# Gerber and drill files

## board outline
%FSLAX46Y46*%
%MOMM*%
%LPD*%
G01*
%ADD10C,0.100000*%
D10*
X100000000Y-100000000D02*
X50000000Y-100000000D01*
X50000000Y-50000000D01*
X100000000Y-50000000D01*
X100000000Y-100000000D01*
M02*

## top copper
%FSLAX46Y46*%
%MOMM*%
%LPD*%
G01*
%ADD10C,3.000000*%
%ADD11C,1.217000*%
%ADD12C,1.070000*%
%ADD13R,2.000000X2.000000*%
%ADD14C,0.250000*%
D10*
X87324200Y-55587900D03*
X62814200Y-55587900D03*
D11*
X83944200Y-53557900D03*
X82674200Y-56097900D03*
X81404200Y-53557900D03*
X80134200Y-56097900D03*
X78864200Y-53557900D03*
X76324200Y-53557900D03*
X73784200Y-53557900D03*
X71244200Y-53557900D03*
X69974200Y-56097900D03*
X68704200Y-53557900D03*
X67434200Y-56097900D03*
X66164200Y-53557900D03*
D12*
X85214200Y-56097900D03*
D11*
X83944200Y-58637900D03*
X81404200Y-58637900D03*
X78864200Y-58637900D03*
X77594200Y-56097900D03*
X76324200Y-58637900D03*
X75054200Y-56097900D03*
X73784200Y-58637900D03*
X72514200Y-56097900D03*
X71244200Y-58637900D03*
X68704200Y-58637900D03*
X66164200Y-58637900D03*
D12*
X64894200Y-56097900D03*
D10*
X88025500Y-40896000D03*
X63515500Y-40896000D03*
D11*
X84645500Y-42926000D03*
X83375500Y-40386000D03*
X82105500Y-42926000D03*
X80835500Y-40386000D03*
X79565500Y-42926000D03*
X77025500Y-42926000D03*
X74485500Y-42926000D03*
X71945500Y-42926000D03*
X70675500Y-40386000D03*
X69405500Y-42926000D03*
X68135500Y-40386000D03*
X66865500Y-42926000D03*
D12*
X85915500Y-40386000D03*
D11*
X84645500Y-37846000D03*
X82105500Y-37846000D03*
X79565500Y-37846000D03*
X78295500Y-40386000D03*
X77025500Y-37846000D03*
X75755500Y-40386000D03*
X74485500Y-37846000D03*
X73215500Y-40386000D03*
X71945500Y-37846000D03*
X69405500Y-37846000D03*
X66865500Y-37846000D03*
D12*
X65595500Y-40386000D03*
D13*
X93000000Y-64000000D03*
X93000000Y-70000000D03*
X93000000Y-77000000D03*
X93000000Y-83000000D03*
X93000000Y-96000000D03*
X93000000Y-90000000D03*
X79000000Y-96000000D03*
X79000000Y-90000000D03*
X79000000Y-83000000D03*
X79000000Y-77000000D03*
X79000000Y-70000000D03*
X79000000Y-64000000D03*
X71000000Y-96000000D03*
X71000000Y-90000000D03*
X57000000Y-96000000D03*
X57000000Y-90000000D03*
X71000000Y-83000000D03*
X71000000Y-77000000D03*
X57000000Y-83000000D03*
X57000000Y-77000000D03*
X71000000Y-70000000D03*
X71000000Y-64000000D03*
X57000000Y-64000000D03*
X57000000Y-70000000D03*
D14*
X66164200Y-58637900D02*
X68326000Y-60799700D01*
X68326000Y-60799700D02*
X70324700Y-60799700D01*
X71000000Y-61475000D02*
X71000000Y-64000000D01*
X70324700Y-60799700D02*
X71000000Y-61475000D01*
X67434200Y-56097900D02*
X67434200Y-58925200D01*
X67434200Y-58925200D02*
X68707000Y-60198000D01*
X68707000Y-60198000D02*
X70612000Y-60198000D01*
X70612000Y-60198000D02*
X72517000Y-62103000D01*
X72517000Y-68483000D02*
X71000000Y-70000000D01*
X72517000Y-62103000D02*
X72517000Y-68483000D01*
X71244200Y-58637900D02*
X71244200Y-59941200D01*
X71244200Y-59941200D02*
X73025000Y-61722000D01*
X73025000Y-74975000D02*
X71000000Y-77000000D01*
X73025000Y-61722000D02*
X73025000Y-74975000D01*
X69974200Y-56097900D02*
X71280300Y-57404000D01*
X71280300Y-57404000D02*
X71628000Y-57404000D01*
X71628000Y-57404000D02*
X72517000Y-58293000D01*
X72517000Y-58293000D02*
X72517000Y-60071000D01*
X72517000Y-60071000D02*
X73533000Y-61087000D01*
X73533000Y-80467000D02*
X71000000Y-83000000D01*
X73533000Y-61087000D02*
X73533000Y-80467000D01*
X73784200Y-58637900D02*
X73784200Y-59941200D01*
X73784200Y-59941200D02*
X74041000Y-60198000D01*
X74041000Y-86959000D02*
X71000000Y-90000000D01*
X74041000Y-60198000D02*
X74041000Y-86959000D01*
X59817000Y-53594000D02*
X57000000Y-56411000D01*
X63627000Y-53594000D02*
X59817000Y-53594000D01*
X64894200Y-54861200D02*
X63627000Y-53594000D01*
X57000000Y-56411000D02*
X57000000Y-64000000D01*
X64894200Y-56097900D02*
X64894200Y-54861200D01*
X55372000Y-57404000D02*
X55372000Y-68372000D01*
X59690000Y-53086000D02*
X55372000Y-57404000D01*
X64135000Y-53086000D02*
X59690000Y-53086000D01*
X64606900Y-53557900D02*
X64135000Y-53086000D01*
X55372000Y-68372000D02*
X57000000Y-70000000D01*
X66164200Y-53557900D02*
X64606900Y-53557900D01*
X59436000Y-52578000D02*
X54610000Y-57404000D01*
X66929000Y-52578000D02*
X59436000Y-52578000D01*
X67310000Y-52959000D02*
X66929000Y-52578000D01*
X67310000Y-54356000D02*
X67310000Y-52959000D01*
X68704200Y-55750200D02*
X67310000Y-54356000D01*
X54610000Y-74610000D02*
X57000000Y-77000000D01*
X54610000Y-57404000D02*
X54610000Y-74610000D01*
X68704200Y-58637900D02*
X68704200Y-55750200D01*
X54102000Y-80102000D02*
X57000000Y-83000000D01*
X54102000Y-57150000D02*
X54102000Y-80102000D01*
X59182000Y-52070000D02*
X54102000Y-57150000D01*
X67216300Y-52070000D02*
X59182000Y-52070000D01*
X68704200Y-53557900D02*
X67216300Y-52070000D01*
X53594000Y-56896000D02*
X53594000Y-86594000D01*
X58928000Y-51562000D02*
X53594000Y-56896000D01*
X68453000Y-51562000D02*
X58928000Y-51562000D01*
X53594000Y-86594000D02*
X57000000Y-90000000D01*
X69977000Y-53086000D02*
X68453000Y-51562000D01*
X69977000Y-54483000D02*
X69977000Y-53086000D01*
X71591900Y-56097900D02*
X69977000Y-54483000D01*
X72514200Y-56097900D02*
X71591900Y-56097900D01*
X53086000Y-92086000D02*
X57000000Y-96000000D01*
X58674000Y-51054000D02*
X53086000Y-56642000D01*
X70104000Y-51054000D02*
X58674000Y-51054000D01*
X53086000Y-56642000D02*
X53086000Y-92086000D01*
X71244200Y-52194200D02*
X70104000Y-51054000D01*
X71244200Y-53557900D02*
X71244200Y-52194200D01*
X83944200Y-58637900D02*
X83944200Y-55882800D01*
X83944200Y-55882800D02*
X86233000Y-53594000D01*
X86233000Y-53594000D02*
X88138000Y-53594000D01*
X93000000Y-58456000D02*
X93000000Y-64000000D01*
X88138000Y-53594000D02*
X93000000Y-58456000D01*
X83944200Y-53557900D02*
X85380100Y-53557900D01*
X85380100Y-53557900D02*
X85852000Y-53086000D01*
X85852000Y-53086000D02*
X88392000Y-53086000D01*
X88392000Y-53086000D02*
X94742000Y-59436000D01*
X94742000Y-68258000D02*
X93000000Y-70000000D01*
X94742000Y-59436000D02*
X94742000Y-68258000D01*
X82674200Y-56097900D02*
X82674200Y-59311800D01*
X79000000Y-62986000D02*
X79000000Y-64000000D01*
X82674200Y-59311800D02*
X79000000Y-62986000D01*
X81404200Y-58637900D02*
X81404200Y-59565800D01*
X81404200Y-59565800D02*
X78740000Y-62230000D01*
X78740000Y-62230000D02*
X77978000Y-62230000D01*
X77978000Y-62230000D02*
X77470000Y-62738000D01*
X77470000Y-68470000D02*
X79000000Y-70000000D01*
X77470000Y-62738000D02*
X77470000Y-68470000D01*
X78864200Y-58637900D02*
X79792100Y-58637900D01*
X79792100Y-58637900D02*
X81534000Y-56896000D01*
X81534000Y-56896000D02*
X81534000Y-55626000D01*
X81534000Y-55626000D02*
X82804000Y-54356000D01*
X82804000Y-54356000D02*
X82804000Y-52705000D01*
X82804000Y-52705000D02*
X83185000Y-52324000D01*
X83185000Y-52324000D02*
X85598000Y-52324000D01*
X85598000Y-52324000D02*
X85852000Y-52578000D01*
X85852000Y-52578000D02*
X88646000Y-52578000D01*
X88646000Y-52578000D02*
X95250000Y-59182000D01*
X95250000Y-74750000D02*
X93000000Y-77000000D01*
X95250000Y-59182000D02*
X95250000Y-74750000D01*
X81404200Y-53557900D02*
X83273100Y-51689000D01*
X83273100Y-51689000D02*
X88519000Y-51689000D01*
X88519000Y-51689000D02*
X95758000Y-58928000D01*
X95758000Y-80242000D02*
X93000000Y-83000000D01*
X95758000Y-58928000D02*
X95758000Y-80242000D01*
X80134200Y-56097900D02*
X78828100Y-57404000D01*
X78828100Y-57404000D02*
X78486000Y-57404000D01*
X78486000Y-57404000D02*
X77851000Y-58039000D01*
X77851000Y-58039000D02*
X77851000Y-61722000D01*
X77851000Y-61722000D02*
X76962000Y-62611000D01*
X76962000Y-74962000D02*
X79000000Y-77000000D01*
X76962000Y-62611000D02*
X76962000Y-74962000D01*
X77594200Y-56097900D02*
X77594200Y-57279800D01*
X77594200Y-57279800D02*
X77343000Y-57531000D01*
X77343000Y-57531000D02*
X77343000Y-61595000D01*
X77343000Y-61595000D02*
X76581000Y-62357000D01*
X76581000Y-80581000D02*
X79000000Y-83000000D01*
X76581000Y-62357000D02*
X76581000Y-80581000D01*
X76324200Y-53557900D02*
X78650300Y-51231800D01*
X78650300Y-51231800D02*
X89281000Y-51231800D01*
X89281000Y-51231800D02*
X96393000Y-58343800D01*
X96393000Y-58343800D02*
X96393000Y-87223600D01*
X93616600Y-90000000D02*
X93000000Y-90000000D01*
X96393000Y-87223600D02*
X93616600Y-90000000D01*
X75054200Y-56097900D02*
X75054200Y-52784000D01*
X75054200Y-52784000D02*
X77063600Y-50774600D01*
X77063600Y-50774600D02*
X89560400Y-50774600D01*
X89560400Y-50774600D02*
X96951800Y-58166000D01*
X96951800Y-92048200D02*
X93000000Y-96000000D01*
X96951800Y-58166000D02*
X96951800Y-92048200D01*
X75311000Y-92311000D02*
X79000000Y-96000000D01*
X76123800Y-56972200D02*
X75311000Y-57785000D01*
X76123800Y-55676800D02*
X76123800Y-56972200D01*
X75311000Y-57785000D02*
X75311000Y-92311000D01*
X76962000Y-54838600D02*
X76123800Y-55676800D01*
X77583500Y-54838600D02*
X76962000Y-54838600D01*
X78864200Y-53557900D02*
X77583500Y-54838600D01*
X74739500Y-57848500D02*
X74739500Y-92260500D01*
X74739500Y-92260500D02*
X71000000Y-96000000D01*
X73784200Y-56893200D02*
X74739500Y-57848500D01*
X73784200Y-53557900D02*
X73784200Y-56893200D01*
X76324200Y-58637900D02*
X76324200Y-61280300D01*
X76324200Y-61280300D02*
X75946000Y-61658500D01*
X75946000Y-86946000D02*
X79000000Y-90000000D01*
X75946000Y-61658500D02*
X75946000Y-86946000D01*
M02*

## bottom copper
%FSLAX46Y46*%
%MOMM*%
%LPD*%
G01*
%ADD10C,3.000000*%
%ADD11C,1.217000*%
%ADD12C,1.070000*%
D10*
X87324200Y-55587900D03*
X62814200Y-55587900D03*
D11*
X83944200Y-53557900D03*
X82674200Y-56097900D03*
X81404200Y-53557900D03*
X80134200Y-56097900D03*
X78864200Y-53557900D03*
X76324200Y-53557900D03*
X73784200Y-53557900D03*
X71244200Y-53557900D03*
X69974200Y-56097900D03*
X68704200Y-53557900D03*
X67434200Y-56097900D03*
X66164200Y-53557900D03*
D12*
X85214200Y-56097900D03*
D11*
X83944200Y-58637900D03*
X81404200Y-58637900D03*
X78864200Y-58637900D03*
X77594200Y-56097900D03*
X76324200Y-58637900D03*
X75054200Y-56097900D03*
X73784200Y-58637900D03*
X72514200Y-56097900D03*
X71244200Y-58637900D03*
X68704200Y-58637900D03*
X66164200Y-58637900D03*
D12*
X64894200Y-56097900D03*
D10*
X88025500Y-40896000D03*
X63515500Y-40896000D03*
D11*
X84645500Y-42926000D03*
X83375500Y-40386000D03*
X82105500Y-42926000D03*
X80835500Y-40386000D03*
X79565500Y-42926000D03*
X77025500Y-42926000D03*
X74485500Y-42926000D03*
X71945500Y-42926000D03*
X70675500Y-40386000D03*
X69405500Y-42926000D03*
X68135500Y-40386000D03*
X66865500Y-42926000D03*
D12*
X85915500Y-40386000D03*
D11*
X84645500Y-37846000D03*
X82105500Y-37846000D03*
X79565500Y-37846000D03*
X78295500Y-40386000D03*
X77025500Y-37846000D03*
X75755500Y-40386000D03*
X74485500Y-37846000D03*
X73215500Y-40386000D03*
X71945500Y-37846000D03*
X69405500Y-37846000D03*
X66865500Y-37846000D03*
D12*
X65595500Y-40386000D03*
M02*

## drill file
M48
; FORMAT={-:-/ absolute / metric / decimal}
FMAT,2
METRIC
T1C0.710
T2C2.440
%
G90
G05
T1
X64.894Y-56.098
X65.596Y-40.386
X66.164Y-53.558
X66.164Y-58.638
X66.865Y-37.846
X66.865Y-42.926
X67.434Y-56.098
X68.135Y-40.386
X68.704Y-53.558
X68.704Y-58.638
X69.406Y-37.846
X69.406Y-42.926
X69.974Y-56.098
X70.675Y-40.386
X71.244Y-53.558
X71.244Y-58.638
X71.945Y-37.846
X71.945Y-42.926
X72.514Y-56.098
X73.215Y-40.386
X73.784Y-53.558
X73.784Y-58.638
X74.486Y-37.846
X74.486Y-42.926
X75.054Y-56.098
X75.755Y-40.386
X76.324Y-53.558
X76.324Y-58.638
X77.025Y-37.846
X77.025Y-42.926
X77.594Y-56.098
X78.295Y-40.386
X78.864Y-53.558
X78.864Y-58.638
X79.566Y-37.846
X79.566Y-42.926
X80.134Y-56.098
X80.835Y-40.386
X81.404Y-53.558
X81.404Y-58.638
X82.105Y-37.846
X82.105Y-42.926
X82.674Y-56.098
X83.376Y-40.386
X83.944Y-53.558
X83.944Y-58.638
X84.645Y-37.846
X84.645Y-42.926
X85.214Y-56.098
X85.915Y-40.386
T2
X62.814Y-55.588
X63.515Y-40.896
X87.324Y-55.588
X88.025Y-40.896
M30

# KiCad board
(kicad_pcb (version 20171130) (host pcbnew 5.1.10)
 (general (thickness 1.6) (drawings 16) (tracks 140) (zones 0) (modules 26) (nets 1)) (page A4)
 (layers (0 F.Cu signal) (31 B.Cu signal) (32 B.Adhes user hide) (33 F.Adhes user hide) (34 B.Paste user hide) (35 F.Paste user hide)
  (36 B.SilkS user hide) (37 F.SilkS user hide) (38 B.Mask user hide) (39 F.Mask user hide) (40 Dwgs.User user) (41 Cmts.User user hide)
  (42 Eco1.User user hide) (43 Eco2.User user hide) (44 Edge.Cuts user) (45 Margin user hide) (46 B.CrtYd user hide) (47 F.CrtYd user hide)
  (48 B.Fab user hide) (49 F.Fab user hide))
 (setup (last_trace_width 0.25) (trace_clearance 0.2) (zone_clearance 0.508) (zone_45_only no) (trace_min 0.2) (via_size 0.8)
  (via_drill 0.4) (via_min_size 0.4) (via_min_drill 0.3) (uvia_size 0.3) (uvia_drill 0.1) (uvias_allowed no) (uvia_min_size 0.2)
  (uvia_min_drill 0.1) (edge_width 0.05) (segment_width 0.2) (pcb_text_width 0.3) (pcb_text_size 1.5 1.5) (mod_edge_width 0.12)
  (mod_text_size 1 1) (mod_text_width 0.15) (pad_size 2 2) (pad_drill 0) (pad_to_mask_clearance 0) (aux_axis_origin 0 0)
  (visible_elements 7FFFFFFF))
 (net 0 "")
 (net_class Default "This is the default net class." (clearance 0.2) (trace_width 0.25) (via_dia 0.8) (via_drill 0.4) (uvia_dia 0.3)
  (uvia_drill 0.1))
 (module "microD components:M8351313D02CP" (layer F.Cu) (at 64.8942 56.0979 180)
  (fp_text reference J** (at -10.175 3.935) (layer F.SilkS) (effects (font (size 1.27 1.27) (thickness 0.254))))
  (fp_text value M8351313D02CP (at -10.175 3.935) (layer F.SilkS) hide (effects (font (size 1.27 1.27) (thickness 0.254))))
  (pad MH2 thru_hole circle (at -22.43 0.51 180) (size 3 3) (drill 2.44) (layers *.Cu *.Mask))
  (pad MH1 thru_hole circle (at 2.08 0.51 180) (size 3 3) (drill 2.44) (layers *.Cu *.Mask))
  (pad 25 thru_hole circle (at -19.05 2.54 180) (size 1.217 1.217) (drill 0.71) (layers *.Cu *.Mask))
  (pad 24 thru_hole circle (at -17.78 0 180) (size 1.217 1.217) (drill 0.71) (layers *.Cu *.Mask))
  (pad 23 thru_hole circle (at -16.51 2.54 180) (size 1.217 1.217) (drill 0.71) (layers *.Cu *.Mask))
  (pad 22 thru_hole circle (at -15.24 0 180) (size 1.217 1.217) (drill 0.71) (layers *.Cu *.Mask))
  (pad 21 thru_hole circle (at -13.97 2.54 180) (size 1.217 1.217) (drill 0.71) (layers *.Cu *.Mask))
  (pad 20 thru_hole circle (at -11.43 2.54 180) (size 1.217 1.217) (drill 0.71) (layers *.Cu *.Mask))
  (pad 19 thru_hole circle (at -8.89 2.54 180) (size 1.217 1.217) (drill 0.71) (layers *.Cu *.Mask))
  (pad 18 thru_hole circle (at -6.35 2.54 180) (size 1.217 1.217) (drill 0.71) (layers *.Cu *.Mask))
  (pad 17 thru_hole circle (at -5.08 0 180) (size 1.217 1.217) (drill 0.71) (layers *.Cu *.Mask))
  (pad 16 thru_hole circle (at -3.81 2.54 180) (size 1.217 1.217) (drill 0.71) (layers *.Cu *.Mask))
  (pad 15 thru_hole circle (at -2.54 0 180) (size 1.217 1.217) (drill 0.71) (layers *.Cu *.Mask))
  (pad 14 thru_hole circle (at -1.27 2.54 180) (size 1.217 1.217) (drill 0.71) (layers *.Cu *.Mask))
  (pad 13 thru_hole circle (at -20.32 0 180) (size 1.07 1.07) (drill 0.71) (layers *.Cu *.Mask))
  (pad 12 thru_hole circle (at -19.05 -2.54 180) (size 1.217 1.217) (drill 0.71) (layers *.Cu *.Mask))
  (pad 11 thru_hole circle (at -16.51 -2.54 180) (size 1.217 1.217) (drill 0.71) (layers *.Cu *.Mask))
  (pad 10 thru_hole circle (at -13.97 -2.54 180) (size 1.217 1.217) (drill 0.71) (layers *.Cu *.Mask))
  (pad 9 thru_hole circle (at -12.7 0 180) (size 1.217 1.217) (drill 0.71) (layers *.Cu *.Mask))
  (pad 8 thru_hole circle (at -11.43 -2.54 180) (size 1.217 1.217) (drill 0.71) (layers *.Cu *.Mask))
  (pad 7 thru_hole circle (at -10.16 0 180) (size 1.217 1.217) (drill 0.71) (layers *.Cu *.Mask))
  (pad 6 thru_hole circle (at -8.89 -2.54 180) (size 1.217 1.217) (drill 0.71) (layers *.Cu *.Mask))
  (pad 5 thru_hole circle (at -7.62 0 180) (size 1.217 1.217) (drill 0.71) (layers *.Cu *.Mask))
  (pad 4 thru_hole circle (at -6.35 -2.54 180) (size 1.217 1.217) (drill 0.71) (layers *.Cu *.Mask))
  (pad 3 thru_hole circle (at -3.81 -2.54 180) (size 1.217 1.217) (drill 0.71) (layers *.Cu *.Mask))
  (pad 2 thru_hole circle (at -1.27 -2.54 180) (size 1.217 1.217) (drill 0.71) (layers *.Cu *.Mask))
  (pad 1 thru_hole circle (at 0 0 180) (size 1.07 1.07) (drill 0.71) (layers *.Cu *.Mask)))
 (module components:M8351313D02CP (layer B.Cu) (at 65.5955 40.386 180)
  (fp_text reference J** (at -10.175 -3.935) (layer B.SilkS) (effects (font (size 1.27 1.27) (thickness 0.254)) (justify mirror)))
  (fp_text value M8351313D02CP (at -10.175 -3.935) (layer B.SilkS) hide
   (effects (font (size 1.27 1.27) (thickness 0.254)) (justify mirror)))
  (pad MH2 thru_hole circle (at -22.43 -0.51 180) (size 3 3) (drill 2.44) (layers *.Cu *.Mask))
  (pad MH1 thru_hole circle (at 2.08 -0.51 180) (size 3 3) (drill 2.44) (layers *.Cu *.Mask))
  (pad 25 thru_hole circle (at -19.05 -2.54 180) (size 1.217 1.217) (drill 0.71) (layers *.Cu *.Mask))
  (pad 24 thru_hole circle (at -17.78 0 180) (size 1.217 1.217) (drill 0.71) (layers *.Cu *.Mask))
  (pad 23 thru_hole circle (at -16.51 -2.54 180) (size 1.217 1.217) (drill 0.71) (layers *.Cu *.Mask))
  (pad 22 thru_hole circle (at -15.24 0 180) (size 1.217 1.217) (drill 0.71) (layers *.Cu *.Mask))
  (pad 21 thru_hole circle (at -13.97 -2.54 180) (size 1.217 1.217) (drill 0.71) (layers *.Cu *.Mask))
  (pad 20 thru_hole circle (at -11.43 -2.54 180) (size 1.217 1.217) (drill 0.71) (layers *.Cu *.Mask))
  (pad 19 thru_hole circle (at -8.89 -2.54 180) (size 1.217 1.217) (drill 0.71) (layers *.Cu *.Mask))
  (pad 18 thru_hole circle (at -6.35 -2.54 180) (size 1.217 1.217) (drill 0.71) (layers *.Cu *.Mask))
  (pad 17 thru_hole circle (at -5.08 0 180) (size 1.217 1.217) (drill 0.71) (layers *.Cu *.Mask))
  (pad 16 thru_hole circle (at -3.81 -2.54 180) (size 1.217 1.217) (drill 0.71) (layers *.Cu *.Mask))
  (pad 15 thru_hole circle (at -2.54 0 180) (size 1.217 1.217) (drill 0.71) (layers *.Cu *.Mask))
  (pad 14 thru_hole circle (at -1.27 -2.54 180) (size 1.217 1.217) (drill 0.71) (layers *.Cu *.Mask))
  (pad 13 thru_hole circle (at -20.32 0 180) (size 1.07 1.07) (drill 0.71) (layers *.Cu *.Mask))
  (pad 12 thru_hole circle (at -19.05 2.54 180) (size 1.217 1.217) (drill 0.71) (layers *.Cu *.Mask))
  (pad 11 thru_hole circle (at -16.51 2.54 180) (size 1.217 1.217) (drill 0.71) (layers *.Cu *.Mask))
  (pad 10 thru_hole circle (at -13.97 2.54 180) (size 1.217 1.217) (drill 0.71) (layers *.Cu *.Mask))
  (pad 9 thru_hole circle (at -12.7 0 180) (size 1.217 1.217) (drill 0.71) (layers *.Cu *.Mask))
  (pad 8 thru_hole circle (at -11.43 2.54 180) (size 1.217 1.217) (drill 0.71) (layers *.Cu *.Mask))
  (pad 7 thru_hole circle (at -10.16 0 180) (size 1.217 1.217) (drill 0.71) (layers *.Cu *.Mask))
  (pad 6 thru_hole circle (at -8.89 2.54 180) (size 1.217 1.217) (drill 0.71) (layers *.Cu *.Mask))
  (pad 5 thru_hole circle (at -7.62 0 180) (size 1.217 1.217) (drill 0.71) (layers *.Cu *.Mask))
  (pad 4 thru_hole circle (at -6.35 2.54 180) (size 1.217 1.217) (drill 0.71) (layers *.Cu *.Mask))
  (pad 3 thru_hole circle (at -3.81 2.54 180) (size 1.217 1.217) (drill 0.71) (layers *.Cu *.Mask))
  (pad 2 thru_hole circle (at -1.27 2.54 180) (size 1.217 1.217) (drill 0.71) (layers *.Cu *.Mask))
  (pad 1 thru_hole circle (at 0 0 180) (size 1.07 1.07) (drill 0.71) (layers *.Cu *.Mask)))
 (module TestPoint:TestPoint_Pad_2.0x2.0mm (layer F.Cu) (at 93 64)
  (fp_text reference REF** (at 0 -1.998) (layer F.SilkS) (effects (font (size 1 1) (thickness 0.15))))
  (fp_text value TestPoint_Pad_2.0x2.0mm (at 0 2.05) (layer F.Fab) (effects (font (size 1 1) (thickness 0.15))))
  (pad 1 smd rect (at 0 0) (size 2 2) (layers F.Cu F.Mask)))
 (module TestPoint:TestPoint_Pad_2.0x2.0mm (layer F.Cu) (at 93 70)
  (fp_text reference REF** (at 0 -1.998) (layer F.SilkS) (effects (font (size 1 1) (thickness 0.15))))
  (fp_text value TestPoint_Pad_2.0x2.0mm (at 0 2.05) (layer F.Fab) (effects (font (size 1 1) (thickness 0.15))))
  (pad 1 smd rect (at 0 0) (size 2 2) (layers F.Cu F.Mask)))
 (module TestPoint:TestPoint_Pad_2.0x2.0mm (layer F.Cu) (at 93 77)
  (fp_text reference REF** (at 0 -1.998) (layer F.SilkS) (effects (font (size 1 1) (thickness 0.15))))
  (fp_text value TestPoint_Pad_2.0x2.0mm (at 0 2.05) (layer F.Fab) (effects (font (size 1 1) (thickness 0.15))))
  (pad 1 smd rect (at 0 0) (size 2 2) (layers F.Cu F.Mask)))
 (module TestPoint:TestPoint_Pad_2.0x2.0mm (layer F.Cu) (at 93 83)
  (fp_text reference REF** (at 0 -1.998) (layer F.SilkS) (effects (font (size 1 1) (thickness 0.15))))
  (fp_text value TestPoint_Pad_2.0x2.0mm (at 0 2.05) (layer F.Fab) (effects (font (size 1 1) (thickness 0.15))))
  (pad 1 smd rect (at 0 0) (size 2 2) (layers F.Cu F.Mask)))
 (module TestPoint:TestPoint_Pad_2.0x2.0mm (layer F.Cu) (at 93 96)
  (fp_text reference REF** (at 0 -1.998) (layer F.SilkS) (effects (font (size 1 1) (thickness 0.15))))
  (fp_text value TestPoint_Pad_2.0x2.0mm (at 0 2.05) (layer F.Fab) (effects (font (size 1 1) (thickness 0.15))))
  (pad 1 smd rect (at 0 0) (size 2 2) (layers F.Cu F.Mask)))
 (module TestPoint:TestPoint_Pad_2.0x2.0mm (layer F.Cu) (at 93 90)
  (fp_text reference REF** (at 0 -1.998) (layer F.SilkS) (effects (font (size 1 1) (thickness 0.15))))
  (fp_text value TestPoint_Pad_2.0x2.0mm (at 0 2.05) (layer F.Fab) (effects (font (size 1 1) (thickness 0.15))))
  (pad 1 smd rect (at 0 0) (size 2 2) (layers F.Cu F.Mask)))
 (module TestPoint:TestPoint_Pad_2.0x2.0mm (layer F.Cu) (at 79 96)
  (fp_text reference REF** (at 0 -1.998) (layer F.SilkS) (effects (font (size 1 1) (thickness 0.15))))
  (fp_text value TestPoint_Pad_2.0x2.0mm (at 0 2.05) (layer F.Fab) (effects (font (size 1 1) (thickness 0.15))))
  (pad 1 smd rect (at 0 0) (size 2 2) (layers F.Cu F.Mask)))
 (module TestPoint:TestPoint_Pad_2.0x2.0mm (layer F.Cu) (at 79 90)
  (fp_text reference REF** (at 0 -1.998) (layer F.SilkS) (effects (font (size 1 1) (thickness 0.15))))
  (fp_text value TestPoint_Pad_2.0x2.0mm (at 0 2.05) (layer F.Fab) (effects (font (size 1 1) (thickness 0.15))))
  (pad 1 smd rect (at 0 0) (size 2 2) (layers F.Cu F.Mask)))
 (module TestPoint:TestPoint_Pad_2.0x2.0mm (layer F.Cu) (at 79 83)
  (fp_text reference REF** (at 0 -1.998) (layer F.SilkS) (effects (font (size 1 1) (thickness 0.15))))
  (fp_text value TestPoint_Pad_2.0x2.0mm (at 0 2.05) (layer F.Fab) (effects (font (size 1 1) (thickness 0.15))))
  (pad 1 smd rect (at 0 0) (size 2 2) (layers F.Cu F.Mask)))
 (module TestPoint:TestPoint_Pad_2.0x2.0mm (layer F.Cu) (at 79 77)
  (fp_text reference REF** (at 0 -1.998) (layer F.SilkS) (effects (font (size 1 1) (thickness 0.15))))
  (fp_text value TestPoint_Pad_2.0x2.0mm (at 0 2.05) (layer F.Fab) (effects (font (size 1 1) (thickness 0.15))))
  (pad 1 smd rect (at 0 0) (size 2 2) (layers F.Cu F.Mask)))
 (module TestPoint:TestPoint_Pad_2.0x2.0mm (layer F.Cu) (at 79 70)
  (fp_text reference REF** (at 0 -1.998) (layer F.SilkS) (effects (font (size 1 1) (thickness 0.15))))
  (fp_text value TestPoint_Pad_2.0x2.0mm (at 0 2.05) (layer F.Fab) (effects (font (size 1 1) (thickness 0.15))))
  (pad 1 smd rect (at 0 0) (size 2 2) (layers F.Cu F.Mask)))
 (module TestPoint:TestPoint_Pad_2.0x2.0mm (layer F.Cu) (at 79 64)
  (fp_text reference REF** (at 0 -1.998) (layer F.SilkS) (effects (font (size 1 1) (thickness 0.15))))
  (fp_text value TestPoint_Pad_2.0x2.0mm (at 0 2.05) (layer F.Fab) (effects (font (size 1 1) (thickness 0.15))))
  (pad 1 smd rect (at 0 0) (size 2 2) (layers F.Cu F.Mask)))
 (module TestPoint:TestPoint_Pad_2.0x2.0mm (layer F.Cu) (at 71 96)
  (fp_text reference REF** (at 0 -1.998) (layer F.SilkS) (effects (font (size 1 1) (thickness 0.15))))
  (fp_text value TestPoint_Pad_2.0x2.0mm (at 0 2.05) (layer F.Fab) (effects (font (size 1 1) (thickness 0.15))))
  (pad 12 smd rect (at 0 0) (size 2 2) (layers F.Cu F.Mask)))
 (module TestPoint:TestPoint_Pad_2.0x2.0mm (layer F.Cu) (at 71 90)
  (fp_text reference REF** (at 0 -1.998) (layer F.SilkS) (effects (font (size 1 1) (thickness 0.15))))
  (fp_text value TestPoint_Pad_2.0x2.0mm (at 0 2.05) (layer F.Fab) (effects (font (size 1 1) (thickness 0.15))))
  (pad 11 smd rect (at 0 0) (size 2 2) (layers F.Cu F.Mask)))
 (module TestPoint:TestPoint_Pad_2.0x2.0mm (layer F.Cu) (at 57 96)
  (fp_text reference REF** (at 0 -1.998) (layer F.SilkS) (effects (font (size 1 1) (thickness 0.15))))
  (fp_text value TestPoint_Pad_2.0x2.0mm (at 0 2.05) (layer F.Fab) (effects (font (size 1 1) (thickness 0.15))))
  (pad 10 smd rect (at 0 0) (size 2 2) (layers F.Cu F.Mask)))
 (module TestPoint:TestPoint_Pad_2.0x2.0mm (layer F.Cu) (at 57 90)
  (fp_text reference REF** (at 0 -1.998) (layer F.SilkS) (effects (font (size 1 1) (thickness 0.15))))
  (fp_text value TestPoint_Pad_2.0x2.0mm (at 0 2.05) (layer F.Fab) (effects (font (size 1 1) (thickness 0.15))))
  (pad 9 smd rect (at 0 0) (size 2 2) (layers F.Cu F.Mask)))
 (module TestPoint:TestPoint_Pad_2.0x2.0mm (layer F.Cu) (at 71 83)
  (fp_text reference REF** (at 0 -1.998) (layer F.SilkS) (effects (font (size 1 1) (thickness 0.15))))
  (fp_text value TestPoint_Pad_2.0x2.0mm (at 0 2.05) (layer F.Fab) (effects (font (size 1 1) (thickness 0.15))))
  (pad 8 smd rect (at 0 0) (size 2 2) (layers F.Cu F.Mask)))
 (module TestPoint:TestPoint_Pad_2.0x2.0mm (layer F.Cu) (at 71 77)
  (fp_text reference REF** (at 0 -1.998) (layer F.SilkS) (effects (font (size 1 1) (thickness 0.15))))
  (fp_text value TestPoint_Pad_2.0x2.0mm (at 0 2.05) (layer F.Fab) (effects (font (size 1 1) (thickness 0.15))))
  (pad 7 smd rect (at 0 0) (size 2 2) (layers F.Cu F.Mask)))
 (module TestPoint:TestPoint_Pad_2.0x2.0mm (layer F.Cu) (at 57 83)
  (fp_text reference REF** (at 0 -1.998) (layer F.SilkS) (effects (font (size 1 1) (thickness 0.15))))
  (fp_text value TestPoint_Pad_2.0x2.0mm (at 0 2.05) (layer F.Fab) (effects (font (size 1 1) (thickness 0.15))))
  (pad 6 smd rect (at 0 0) (size 2 2) (layers F.Cu F.Mask)))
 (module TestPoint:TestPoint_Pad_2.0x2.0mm (layer F.Cu) (at 57 77)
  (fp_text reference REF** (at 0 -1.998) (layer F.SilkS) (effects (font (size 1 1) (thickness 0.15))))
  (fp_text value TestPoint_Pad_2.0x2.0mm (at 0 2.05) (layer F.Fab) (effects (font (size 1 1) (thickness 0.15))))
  (pad 5 smd rect (at 0 0) (size 2 2) (layers F.Cu F.Mask)))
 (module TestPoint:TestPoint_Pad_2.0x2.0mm (layer F.Cu) (at 71 70)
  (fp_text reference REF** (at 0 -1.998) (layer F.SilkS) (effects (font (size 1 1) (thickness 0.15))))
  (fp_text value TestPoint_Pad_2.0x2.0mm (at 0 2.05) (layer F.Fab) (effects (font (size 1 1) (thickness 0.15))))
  (pad 4 smd rect (at 0 0) (size 2 2) (layers F.Cu F.Mask)))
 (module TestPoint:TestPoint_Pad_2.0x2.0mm (layer F.Cu) (at 71 64)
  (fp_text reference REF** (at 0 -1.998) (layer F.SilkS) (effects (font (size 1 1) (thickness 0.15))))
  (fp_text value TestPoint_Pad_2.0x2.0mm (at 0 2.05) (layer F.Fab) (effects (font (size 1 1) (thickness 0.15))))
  (pad 3 smd rect (at 0 0) (size 2 2) (layers F.Cu F.Mask)))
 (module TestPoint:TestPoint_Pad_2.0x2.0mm (layer F.Cu) (at 57 64)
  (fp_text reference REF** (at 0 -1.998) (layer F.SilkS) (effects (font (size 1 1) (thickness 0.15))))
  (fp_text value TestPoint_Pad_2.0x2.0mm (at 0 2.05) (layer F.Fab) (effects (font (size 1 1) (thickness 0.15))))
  (pad 1 smd rect (at 0 0) (size 2 2) (layers F.Cu F.Mask)))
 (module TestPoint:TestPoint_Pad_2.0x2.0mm (layer F.Cu) (at 57 70)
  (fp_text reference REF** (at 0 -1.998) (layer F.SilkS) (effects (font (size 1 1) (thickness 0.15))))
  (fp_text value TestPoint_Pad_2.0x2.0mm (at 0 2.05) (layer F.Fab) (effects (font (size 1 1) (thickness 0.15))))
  (pad 2 smd rect (at 0 0) (size 2 2) (layers F.Cu F.Mask)))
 (gr_poly (pts (xy 100 100) (xy 50 100) (xy 50 50) (xy 100 50)) (layer Edge.Cuts) (width 0.1))
 (segment (start 66.1642 58.6379) (end 68.326 60.7997) (width 0.25) (layer F.Cu) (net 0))
 (segment (start 68.326 60.7997) (end 70.3247 60.7997) (width 0.25) (layer F.Cu) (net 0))
 (segment (start 71 61.475) (end 71 64) (width 0.25) (layer F.Cu) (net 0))
 (segment (start 70.3247 60.7997) (end 71 61.475) (width 0.25) (layer F.Cu) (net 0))
 (segment (start 67.4342 56.0979) (end 67.4342 58.9252) (width 0.25) (layer F.Cu) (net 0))
 (segment (start 67.4342 58.9252) (end 68.707 60.198) (width 0.25) (layer F.Cu) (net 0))
 (segment (start 68.707 60.198) (end 70.612 60.198) (width 0.25) (layer F.Cu) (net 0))
 (segment (start 70.612 60.198) (end 72.517 62.103) (width 0.25) (layer F.Cu) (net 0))
 (segment (start 72.517 68.483) (end 71 70) (width 0.25) (layer F.Cu) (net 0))
 (segment (start 72.517 62.103) (end 72.517 68.483) (width 0.25) (layer F.Cu) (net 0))
 (segment (start 71.2442 58.6379) (end 71.2442 59.9412) (width 0.25) (layer F.Cu) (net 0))
 (segment (start 71.2442 59.9412) (end 73.025 61.722) (width 0.25) (layer F.Cu) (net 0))
 (segment (start 73.025 74.975) (end 71 77) (width 0.25) (layer F.Cu) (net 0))
 (segment (start 73.025 61.722) (end 73.025 74.975) (width 0.25) (layer F.Cu) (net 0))
 (segment (start 69.9742 56.0979) (end 71.2803 57.404) (width 0.25) (layer F.Cu) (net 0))
 (segment (start 71.2803 57.404) (end 71.628 57.404) (width 0.25) (layer F.Cu) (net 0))
 (segment (start 71.628 57.404) (end 72.517 58.293) (width 0.25) (layer F.Cu) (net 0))
 (segment (start 72.517 58.293) (end 72.517 60.071) (width 0.25) (layer F.Cu) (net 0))
 (segment (start 72.517 60.071) (end 73.533 61.087) (width 0.25) (layer F.Cu) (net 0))
 (segment (start 73.533 80.467) (end 71 83) (width 0.25) (layer F.Cu) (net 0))
 (segment (start 73.533 61.087) (end 73.533 80.467) (width 0.25) (layer F.Cu) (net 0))
 (segment (start 73.7842 58.6379) (end 73.7842 59.9412) (width 0.25) (layer F.Cu) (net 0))
 (segment (start 73.7842 59.9412) (end 74.041 60.198) (width 0.25) (layer F.Cu) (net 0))
 (segment (start 74.041 86.959) (end 71 90) (width 0.25) (layer F.Cu) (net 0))
 (segment (start 74.041 60.198) (end 74.041 86.959) (width 0.25) (layer F.Cu) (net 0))
 (segment (start 59.817 53.594) (end 57 56.411) (width 0.25) (layer F.Cu) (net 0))
 (segment (start 63.627 53.594) (end 59.817 53.594) (width 0.25) (layer F.Cu) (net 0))
 (segment (start 64.8942 54.8612) (end 63.627 53.594) (width 0.25) (layer F.Cu) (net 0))
 (segment (start 57 56.411) (end 57 64) (width 0.25) (layer F.Cu) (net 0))
 (segment (start 64.8942 56.0979) (end 64.8942 54.8612) (width 0.25) (layer F.Cu) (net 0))
 (segment (start 55.372 57.404) (end 55.372 68.372) (width 0.25) (layer F.Cu) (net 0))
 (segment (start 59.69 53.086) (end 55.372 57.404) (width 0.25) (layer F.Cu) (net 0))
 (segment (start 64.135 53.086) (end 59.69 53.086) (width 0.25) (layer F.Cu) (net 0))
 (segment (start 64.6069 53.5579) (end 64.135 53.086) (width 0.25) (layer F.Cu) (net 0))
 (segment (start 55.372 68.372) (end 57 70) (width 0.25) (layer F.Cu) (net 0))
 (segment (start 66.1642 53.5579) (end 64.6069 53.5579) (width 0.25) (layer F.Cu) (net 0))
 (segment (start 59.436 52.578) (end 54.61 57.404) (width 0.25) (layer F.Cu) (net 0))
 (segment (start 66.929 52.578) (end 59.436 52.578) (width 0.25) (layer F.Cu) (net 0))
 (segment (start 67.31 52.959) (end 66.929 52.578) (width 0.25) (layer F.Cu) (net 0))
 (segment (start 67.31 54.356) (end 67.31 52.959) (width 0.25) (layer F.Cu) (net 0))
 (segment (start 68.7042 55.7502) (end 67.31 54.356) (width 0.25) (layer F.Cu) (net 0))
 (segment (start 54.61 74.61) (end 57 77) (width 0.25) (layer F.Cu) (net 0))
 (segment (start 54.61 57.404) (end 54.61 74.61) (width 0.25) (layer F.Cu) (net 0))
 (segment (start 68.7042 58.6379) (end 68.7042 55.7502) (width 0.25) (layer F.Cu) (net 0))
 (segment (start 54.102 80.102) (end 57 83) (width 0.25) (layer F.Cu) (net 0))
 (segment (start 54.102 57.15) (end 54.102 80.102) (width 0.25) (layer F.Cu) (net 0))
 (segment (start 59.182 52.07) (end 54.102 57.15) (width 0.25) (layer F.Cu) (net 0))
 (segment (start 67.2163 52.07) (end 59.182 52.07) (width 0.25) (layer F.Cu) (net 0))
 (segment (start 68.7042 53.5579) (end 67.2163 52.07) (width 0.25) (layer F.Cu) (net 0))
 (segment (start 53.594 56.896) (end 53.594 86.594) (width 0.25) (layer F.Cu) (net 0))
 (segment (start 58.928 51.562) (end 53.594 56.896) (width 0.25) (layer F.Cu) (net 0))
 (segment (start 68.453 51.562) (end 58.928 51.562) (width 0.25) (layer F.Cu) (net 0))
 (segment (start 53.594 86.594) (end 57 90) (width 0.25) (layer F.Cu) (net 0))
 (segment (start 69.977 53.086) (end 68.453 51.562) (width 0.25) (layer F.Cu) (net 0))
 (segment (start 69.977 54.483) (end 69.977 53.086) (width 0.25) (layer F.Cu) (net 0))
 (segment (start 71.5919 56.0979) (end 69.977 54.483) (width 0.25) (layer F.Cu) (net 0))
 (segment (start 72.5142 56.0979) (end 71.5919 56.0979) (width 0.25) (layer F.Cu) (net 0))
 (segment (start 53.086 92.086) (end 57 96) (width 0.25) (layer F.Cu) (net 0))
 (segment (start 58.674 51.054) (end 53.086 56.642) (width 0.25) (layer F.Cu) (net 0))
 (segment (start 70.104 51.054) (end 58.674 51.054) (width 0.25) (layer F.Cu) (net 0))
 (segment (start 53.086 56.642) (end 53.086 92.086) (width 0.25) (layer F.Cu) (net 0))
 (segment (start 71.2442 52.1942) (end 70.104 51.054) (width 0.25) (layer F.Cu) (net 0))
 (segment (start 71.2442 53.5579) (end 71.2442 52.1942) (width 0.25) (layer F.Cu) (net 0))
 (segment (start 83.9442 58.6379) (end 83.9442 55.8828) (width 0.25) (layer F.Cu) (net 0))
 (segment (start 83.9442 55.8828) (end 86.233 53.594) (width 0.25) (layer F.Cu) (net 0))
 (segment (start 86.233 53.594) (end 88.138 53.594) (width 0.25) (layer F.Cu) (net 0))
 (segment (start 93 58.456) (end 93 64) (width 0.25) (layer F.Cu) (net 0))
 (segment (start 88.138 53.594) (end 93 58.456) (width 0.25) (layer F.Cu) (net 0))
 (segment (start 83.9442 53.5579) (end 85.3801 53.5579) (width 0.25) (layer F.Cu) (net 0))
 (segment (start 85.3801 53.5579) (end 85.852 53.086) (width 0.25) (layer F.Cu) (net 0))
 (segment (start 85.852 53.086) (end 88.392 53.086) (width 0.25) (layer F.Cu) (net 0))
 (segment (start 88.392 53.086) (end 94.742 59.436) (width 0.25) (layer F.Cu) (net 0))
 (segment (start 94.742 68.258) (end 93 70) (width 0.25) (layer F.Cu) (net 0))
 (segment (start 94.742 59.436) (end 94.742 68.258) (width 0.25) (layer F.Cu) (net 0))
 (segment (start 82.6742 56.0979) (end 82.6742 59.3118) (width 0.25) (layer F.Cu) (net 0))
 (segment (start 79 62.986) (end 79 64) (width 0.25) (layer F.Cu) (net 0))
 (segment (start 82.6742 59.3118) (end 79 62.986) (width 0.25) (layer F.Cu) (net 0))
 (segment (start 81.4042 58.6379) (end 81.4042 59.5658) (width 0.25) (layer F.Cu) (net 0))
 (segment (start 81.4042 59.5658) (end 78.74 62.23) (width 0.25) (layer F.Cu) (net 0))
 (segment (start 78.74 62.23) (end 77.978 62.23) (width 0.25) (layer F.Cu) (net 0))
 (segment (start 77.978 62.23) (end 77.47 62.738) (width 0.25) (layer F.Cu) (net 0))
 (segment (start 77.47 68.47) (end 79 70) (width 0.25) (layer F.Cu) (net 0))
 (segment (start 77.47 62.738) (end 77.47 68.47) (width 0.25) (layer F.Cu) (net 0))
 (segment (start 78.8642 58.6379) (end 79.7921 58.6379) (width 0.25) (layer F.Cu) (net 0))
 (segment (start 79.7921 58.6379) (end 81.534 56.896) (width 0.25) (layer F.Cu) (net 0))
 (segment (start 81.534 56.896) (end 81.534 55.626) (width 0.25) (layer F.Cu) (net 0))
 (segment (start 81.534 55.626) (end 82.804 54.356) (width 0.25) (layer F.Cu) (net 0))
 (segment (start 82.804 54.356) (end 82.804 52.705) (width 0.25) (layer F.Cu) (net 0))
 (segment (start 82.804 52.705) (end 83.185 52.324) (width 0.25) (layer F.Cu) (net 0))
 (segment (start 83.185 52.324) (end 85.598 52.324) (width 0.25) (layer F.Cu) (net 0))
 (segment (start 85.598 52.324) (end 85.852 52.578) (width 0.25) (layer F.Cu) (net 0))
 (segment (start 85.852 52.578) (end 88.646 52.578) (width 0.25) (layer F.Cu) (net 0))
 (segment (start 88.646 52.578) (end 95.25 59.182) (width 0.25) (layer F.Cu) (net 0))
 (segment (start 95.25 74.75) (end 93 77) (width 0.25) (layer F.Cu) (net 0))
 (segment (start 95.25 59.182) (end 95.25 74.75) (width 0.25) (layer F.Cu) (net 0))
 (segment (start 81.4042 53.5579) (end 83.2731 51.689) (width 0.25) (layer F.Cu) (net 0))
 (segment (start 83.2731 51.689) (end 88.519 51.689) (width 0.25) (layer F.Cu) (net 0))
 (segment (start 88.519 51.689) (end 95.758 58.928) (width 0.25) (layer F.Cu) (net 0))
 (segment (start 95.758 80.242) (end 93 83) (width 0.25) (layer F.Cu) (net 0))
 (segment (start 95.758 58.928) (end 95.758 80.242) (width 0.25) (layer F.Cu) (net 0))
 (segment (start 80.1342 56.0979) (end 78.8281 57.404) (width 0.25) (layer F.Cu) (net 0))
 (segment (start 78.8281 57.404) (end 78.486 57.404) (width 0.25) (layer F.Cu) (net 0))
 (segment (start 78.486 57.404) (end 77.851 58.039) (width 0.25) (layer F.Cu) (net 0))
 (segment (start 77.851 58.039) (end 77.851 61.722) (width 0.25) (layer F.Cu) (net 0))
 (segment (start 77.851 61.722) (end 76.962 62.611) (width 0.25) (layer F.Cu) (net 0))
 (segment (start 76.962 74.962) (end 79 77) (width 0.25) (layer F.Cu) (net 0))
 (segment (start 76.962 62.611) (end 76.962 74.962) (width 0.25) (layer F.Cu) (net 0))
 (segment (start 77.5942 56.0979) (end 77.5942 57.2798) (width 0.25) (layer F.Cu) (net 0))
 (segment (start 77.5942 57.2798) (end 77.343 57.531) (width 0.25) (layer F.Cu) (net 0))
 (segment (start 77.343 57.531) (end 77.343 61.595) (width 0.25) (layer F.Cu) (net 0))
 (segment (start 77.343 61.595) (end 76.581 62.357) (width 0.25) (layer F.Cu) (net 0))
 (segment (start 76.581 80.581) (end 79 83) (width 0.25) (layer F.Cu) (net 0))
 (segment (start 76.581 62.357) (end 76.581 80.581) (width 0.25) (layer F.Cu) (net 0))
 (segment (start 76.3242 53.5579) (end 78.6503 51.2318) (width 0.25) (layer F.Cu) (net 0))
 (segment (start 78.6503 51.2318) (end 89.281 51.2318) (width 0.25) (layer F.Cu) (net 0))
 (segment (start 89.281 51.2318) (end 96.393 58.3438) (width 0.25) (layer F.Cu) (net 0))
 (segment (start 96.393 58.3438) (end 96.393 87.2236) (width 0.25) (layer F.Cu) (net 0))
 (segment (start 93.6166 90) (end 93 90) (width 0.25) (layer F.Cu) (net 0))
 (segment (start 96.393 87.2236) (end 93.6166 90) (width 0.25) (layer F.Cu) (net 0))
 (segment (start 75.0542 56.0979) (end 75.0542 52.784) (width 0.25) (layer F.Cu) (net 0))
 (segment (start 75.0542 52.784) (end 77.0636 50.7746) (width 0.25) (layer F.Cu) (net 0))
 (segment (start 77.0636 50.7746) (end 89.5604 50.7746) (width 0.25) (layer F.Cu) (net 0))
 (segment (start 89.5604 50.7746) (end 96.9518 58.166) (width 0.25) (layer F.Cu) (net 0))
 (segment (start 96.9518 92.0482) (end 93 96) (width 0.25) (layer F.Cu) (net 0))
 (segment (start 96.9518 58.166) (end 96.9518 92.0482) (width 0.25) (layer F.Cu) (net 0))
 (segment (start 75.311 92.311) (end 79 96) (width 0.25) (layer F.Cu) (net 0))
 (segment (start 76.1238 56.9722) (end 75.311 57.785) (width 0.25) (layer F.Cu) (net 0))
 (segment (start 76.1238 55.6768) (end 76.1238 56.9722) (width 0.25) (layer F.Cu) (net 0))
 (segment (start 75.311 57.785) (end 75.311 92.311) (width 0.25) (layer F.Cu) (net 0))
 (segment (start 76.962 54.8386) (end 76.1238 55.6768) (width 0.25) (layer F.Cu) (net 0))
 (segment (start 77.5835 54.8386) (end 76.962 54.8386) (width 0.25) (layer F.Cu) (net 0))
 (segment (start 78.8642 53.5579) (end 77.5835 54.8386) (width 0.25) (layer F.Cu) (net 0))
 (segment (start 74.7395 57.8485) (end 74.7395 92.2605) (width 0.25) (layer F.Cu) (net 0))
 (segment (start 74.7395 92.2605) (end 71 96) (width 0.25) (layer F.Cu) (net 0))
 (segment (start 73.7842 56.8932) (end 74.7395 57.8485) (width 0.25) (layer F.Cu) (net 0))
 (segment (start 73.7842 53.5579) (end 73.7842 56.8932) (width 0.25) (layer F.Cu) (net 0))
 (segment (start 76.3242 58.6379) (end 76.3242 61.2803) (width 0.25) (layer F.Cu) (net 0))
 (segment (start 76.3242 61.2803) (end 75.946 61.6585) (width 0.25) (layer F.Cu) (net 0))
 (segment (start 75.946 86.946) (end 79 90) (width 0.25) (layer F.Cu) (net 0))
 (segment (start 75.946 61.6585) (end 75.946 86.946) (width 0.25) (layer F.Cu) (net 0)))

